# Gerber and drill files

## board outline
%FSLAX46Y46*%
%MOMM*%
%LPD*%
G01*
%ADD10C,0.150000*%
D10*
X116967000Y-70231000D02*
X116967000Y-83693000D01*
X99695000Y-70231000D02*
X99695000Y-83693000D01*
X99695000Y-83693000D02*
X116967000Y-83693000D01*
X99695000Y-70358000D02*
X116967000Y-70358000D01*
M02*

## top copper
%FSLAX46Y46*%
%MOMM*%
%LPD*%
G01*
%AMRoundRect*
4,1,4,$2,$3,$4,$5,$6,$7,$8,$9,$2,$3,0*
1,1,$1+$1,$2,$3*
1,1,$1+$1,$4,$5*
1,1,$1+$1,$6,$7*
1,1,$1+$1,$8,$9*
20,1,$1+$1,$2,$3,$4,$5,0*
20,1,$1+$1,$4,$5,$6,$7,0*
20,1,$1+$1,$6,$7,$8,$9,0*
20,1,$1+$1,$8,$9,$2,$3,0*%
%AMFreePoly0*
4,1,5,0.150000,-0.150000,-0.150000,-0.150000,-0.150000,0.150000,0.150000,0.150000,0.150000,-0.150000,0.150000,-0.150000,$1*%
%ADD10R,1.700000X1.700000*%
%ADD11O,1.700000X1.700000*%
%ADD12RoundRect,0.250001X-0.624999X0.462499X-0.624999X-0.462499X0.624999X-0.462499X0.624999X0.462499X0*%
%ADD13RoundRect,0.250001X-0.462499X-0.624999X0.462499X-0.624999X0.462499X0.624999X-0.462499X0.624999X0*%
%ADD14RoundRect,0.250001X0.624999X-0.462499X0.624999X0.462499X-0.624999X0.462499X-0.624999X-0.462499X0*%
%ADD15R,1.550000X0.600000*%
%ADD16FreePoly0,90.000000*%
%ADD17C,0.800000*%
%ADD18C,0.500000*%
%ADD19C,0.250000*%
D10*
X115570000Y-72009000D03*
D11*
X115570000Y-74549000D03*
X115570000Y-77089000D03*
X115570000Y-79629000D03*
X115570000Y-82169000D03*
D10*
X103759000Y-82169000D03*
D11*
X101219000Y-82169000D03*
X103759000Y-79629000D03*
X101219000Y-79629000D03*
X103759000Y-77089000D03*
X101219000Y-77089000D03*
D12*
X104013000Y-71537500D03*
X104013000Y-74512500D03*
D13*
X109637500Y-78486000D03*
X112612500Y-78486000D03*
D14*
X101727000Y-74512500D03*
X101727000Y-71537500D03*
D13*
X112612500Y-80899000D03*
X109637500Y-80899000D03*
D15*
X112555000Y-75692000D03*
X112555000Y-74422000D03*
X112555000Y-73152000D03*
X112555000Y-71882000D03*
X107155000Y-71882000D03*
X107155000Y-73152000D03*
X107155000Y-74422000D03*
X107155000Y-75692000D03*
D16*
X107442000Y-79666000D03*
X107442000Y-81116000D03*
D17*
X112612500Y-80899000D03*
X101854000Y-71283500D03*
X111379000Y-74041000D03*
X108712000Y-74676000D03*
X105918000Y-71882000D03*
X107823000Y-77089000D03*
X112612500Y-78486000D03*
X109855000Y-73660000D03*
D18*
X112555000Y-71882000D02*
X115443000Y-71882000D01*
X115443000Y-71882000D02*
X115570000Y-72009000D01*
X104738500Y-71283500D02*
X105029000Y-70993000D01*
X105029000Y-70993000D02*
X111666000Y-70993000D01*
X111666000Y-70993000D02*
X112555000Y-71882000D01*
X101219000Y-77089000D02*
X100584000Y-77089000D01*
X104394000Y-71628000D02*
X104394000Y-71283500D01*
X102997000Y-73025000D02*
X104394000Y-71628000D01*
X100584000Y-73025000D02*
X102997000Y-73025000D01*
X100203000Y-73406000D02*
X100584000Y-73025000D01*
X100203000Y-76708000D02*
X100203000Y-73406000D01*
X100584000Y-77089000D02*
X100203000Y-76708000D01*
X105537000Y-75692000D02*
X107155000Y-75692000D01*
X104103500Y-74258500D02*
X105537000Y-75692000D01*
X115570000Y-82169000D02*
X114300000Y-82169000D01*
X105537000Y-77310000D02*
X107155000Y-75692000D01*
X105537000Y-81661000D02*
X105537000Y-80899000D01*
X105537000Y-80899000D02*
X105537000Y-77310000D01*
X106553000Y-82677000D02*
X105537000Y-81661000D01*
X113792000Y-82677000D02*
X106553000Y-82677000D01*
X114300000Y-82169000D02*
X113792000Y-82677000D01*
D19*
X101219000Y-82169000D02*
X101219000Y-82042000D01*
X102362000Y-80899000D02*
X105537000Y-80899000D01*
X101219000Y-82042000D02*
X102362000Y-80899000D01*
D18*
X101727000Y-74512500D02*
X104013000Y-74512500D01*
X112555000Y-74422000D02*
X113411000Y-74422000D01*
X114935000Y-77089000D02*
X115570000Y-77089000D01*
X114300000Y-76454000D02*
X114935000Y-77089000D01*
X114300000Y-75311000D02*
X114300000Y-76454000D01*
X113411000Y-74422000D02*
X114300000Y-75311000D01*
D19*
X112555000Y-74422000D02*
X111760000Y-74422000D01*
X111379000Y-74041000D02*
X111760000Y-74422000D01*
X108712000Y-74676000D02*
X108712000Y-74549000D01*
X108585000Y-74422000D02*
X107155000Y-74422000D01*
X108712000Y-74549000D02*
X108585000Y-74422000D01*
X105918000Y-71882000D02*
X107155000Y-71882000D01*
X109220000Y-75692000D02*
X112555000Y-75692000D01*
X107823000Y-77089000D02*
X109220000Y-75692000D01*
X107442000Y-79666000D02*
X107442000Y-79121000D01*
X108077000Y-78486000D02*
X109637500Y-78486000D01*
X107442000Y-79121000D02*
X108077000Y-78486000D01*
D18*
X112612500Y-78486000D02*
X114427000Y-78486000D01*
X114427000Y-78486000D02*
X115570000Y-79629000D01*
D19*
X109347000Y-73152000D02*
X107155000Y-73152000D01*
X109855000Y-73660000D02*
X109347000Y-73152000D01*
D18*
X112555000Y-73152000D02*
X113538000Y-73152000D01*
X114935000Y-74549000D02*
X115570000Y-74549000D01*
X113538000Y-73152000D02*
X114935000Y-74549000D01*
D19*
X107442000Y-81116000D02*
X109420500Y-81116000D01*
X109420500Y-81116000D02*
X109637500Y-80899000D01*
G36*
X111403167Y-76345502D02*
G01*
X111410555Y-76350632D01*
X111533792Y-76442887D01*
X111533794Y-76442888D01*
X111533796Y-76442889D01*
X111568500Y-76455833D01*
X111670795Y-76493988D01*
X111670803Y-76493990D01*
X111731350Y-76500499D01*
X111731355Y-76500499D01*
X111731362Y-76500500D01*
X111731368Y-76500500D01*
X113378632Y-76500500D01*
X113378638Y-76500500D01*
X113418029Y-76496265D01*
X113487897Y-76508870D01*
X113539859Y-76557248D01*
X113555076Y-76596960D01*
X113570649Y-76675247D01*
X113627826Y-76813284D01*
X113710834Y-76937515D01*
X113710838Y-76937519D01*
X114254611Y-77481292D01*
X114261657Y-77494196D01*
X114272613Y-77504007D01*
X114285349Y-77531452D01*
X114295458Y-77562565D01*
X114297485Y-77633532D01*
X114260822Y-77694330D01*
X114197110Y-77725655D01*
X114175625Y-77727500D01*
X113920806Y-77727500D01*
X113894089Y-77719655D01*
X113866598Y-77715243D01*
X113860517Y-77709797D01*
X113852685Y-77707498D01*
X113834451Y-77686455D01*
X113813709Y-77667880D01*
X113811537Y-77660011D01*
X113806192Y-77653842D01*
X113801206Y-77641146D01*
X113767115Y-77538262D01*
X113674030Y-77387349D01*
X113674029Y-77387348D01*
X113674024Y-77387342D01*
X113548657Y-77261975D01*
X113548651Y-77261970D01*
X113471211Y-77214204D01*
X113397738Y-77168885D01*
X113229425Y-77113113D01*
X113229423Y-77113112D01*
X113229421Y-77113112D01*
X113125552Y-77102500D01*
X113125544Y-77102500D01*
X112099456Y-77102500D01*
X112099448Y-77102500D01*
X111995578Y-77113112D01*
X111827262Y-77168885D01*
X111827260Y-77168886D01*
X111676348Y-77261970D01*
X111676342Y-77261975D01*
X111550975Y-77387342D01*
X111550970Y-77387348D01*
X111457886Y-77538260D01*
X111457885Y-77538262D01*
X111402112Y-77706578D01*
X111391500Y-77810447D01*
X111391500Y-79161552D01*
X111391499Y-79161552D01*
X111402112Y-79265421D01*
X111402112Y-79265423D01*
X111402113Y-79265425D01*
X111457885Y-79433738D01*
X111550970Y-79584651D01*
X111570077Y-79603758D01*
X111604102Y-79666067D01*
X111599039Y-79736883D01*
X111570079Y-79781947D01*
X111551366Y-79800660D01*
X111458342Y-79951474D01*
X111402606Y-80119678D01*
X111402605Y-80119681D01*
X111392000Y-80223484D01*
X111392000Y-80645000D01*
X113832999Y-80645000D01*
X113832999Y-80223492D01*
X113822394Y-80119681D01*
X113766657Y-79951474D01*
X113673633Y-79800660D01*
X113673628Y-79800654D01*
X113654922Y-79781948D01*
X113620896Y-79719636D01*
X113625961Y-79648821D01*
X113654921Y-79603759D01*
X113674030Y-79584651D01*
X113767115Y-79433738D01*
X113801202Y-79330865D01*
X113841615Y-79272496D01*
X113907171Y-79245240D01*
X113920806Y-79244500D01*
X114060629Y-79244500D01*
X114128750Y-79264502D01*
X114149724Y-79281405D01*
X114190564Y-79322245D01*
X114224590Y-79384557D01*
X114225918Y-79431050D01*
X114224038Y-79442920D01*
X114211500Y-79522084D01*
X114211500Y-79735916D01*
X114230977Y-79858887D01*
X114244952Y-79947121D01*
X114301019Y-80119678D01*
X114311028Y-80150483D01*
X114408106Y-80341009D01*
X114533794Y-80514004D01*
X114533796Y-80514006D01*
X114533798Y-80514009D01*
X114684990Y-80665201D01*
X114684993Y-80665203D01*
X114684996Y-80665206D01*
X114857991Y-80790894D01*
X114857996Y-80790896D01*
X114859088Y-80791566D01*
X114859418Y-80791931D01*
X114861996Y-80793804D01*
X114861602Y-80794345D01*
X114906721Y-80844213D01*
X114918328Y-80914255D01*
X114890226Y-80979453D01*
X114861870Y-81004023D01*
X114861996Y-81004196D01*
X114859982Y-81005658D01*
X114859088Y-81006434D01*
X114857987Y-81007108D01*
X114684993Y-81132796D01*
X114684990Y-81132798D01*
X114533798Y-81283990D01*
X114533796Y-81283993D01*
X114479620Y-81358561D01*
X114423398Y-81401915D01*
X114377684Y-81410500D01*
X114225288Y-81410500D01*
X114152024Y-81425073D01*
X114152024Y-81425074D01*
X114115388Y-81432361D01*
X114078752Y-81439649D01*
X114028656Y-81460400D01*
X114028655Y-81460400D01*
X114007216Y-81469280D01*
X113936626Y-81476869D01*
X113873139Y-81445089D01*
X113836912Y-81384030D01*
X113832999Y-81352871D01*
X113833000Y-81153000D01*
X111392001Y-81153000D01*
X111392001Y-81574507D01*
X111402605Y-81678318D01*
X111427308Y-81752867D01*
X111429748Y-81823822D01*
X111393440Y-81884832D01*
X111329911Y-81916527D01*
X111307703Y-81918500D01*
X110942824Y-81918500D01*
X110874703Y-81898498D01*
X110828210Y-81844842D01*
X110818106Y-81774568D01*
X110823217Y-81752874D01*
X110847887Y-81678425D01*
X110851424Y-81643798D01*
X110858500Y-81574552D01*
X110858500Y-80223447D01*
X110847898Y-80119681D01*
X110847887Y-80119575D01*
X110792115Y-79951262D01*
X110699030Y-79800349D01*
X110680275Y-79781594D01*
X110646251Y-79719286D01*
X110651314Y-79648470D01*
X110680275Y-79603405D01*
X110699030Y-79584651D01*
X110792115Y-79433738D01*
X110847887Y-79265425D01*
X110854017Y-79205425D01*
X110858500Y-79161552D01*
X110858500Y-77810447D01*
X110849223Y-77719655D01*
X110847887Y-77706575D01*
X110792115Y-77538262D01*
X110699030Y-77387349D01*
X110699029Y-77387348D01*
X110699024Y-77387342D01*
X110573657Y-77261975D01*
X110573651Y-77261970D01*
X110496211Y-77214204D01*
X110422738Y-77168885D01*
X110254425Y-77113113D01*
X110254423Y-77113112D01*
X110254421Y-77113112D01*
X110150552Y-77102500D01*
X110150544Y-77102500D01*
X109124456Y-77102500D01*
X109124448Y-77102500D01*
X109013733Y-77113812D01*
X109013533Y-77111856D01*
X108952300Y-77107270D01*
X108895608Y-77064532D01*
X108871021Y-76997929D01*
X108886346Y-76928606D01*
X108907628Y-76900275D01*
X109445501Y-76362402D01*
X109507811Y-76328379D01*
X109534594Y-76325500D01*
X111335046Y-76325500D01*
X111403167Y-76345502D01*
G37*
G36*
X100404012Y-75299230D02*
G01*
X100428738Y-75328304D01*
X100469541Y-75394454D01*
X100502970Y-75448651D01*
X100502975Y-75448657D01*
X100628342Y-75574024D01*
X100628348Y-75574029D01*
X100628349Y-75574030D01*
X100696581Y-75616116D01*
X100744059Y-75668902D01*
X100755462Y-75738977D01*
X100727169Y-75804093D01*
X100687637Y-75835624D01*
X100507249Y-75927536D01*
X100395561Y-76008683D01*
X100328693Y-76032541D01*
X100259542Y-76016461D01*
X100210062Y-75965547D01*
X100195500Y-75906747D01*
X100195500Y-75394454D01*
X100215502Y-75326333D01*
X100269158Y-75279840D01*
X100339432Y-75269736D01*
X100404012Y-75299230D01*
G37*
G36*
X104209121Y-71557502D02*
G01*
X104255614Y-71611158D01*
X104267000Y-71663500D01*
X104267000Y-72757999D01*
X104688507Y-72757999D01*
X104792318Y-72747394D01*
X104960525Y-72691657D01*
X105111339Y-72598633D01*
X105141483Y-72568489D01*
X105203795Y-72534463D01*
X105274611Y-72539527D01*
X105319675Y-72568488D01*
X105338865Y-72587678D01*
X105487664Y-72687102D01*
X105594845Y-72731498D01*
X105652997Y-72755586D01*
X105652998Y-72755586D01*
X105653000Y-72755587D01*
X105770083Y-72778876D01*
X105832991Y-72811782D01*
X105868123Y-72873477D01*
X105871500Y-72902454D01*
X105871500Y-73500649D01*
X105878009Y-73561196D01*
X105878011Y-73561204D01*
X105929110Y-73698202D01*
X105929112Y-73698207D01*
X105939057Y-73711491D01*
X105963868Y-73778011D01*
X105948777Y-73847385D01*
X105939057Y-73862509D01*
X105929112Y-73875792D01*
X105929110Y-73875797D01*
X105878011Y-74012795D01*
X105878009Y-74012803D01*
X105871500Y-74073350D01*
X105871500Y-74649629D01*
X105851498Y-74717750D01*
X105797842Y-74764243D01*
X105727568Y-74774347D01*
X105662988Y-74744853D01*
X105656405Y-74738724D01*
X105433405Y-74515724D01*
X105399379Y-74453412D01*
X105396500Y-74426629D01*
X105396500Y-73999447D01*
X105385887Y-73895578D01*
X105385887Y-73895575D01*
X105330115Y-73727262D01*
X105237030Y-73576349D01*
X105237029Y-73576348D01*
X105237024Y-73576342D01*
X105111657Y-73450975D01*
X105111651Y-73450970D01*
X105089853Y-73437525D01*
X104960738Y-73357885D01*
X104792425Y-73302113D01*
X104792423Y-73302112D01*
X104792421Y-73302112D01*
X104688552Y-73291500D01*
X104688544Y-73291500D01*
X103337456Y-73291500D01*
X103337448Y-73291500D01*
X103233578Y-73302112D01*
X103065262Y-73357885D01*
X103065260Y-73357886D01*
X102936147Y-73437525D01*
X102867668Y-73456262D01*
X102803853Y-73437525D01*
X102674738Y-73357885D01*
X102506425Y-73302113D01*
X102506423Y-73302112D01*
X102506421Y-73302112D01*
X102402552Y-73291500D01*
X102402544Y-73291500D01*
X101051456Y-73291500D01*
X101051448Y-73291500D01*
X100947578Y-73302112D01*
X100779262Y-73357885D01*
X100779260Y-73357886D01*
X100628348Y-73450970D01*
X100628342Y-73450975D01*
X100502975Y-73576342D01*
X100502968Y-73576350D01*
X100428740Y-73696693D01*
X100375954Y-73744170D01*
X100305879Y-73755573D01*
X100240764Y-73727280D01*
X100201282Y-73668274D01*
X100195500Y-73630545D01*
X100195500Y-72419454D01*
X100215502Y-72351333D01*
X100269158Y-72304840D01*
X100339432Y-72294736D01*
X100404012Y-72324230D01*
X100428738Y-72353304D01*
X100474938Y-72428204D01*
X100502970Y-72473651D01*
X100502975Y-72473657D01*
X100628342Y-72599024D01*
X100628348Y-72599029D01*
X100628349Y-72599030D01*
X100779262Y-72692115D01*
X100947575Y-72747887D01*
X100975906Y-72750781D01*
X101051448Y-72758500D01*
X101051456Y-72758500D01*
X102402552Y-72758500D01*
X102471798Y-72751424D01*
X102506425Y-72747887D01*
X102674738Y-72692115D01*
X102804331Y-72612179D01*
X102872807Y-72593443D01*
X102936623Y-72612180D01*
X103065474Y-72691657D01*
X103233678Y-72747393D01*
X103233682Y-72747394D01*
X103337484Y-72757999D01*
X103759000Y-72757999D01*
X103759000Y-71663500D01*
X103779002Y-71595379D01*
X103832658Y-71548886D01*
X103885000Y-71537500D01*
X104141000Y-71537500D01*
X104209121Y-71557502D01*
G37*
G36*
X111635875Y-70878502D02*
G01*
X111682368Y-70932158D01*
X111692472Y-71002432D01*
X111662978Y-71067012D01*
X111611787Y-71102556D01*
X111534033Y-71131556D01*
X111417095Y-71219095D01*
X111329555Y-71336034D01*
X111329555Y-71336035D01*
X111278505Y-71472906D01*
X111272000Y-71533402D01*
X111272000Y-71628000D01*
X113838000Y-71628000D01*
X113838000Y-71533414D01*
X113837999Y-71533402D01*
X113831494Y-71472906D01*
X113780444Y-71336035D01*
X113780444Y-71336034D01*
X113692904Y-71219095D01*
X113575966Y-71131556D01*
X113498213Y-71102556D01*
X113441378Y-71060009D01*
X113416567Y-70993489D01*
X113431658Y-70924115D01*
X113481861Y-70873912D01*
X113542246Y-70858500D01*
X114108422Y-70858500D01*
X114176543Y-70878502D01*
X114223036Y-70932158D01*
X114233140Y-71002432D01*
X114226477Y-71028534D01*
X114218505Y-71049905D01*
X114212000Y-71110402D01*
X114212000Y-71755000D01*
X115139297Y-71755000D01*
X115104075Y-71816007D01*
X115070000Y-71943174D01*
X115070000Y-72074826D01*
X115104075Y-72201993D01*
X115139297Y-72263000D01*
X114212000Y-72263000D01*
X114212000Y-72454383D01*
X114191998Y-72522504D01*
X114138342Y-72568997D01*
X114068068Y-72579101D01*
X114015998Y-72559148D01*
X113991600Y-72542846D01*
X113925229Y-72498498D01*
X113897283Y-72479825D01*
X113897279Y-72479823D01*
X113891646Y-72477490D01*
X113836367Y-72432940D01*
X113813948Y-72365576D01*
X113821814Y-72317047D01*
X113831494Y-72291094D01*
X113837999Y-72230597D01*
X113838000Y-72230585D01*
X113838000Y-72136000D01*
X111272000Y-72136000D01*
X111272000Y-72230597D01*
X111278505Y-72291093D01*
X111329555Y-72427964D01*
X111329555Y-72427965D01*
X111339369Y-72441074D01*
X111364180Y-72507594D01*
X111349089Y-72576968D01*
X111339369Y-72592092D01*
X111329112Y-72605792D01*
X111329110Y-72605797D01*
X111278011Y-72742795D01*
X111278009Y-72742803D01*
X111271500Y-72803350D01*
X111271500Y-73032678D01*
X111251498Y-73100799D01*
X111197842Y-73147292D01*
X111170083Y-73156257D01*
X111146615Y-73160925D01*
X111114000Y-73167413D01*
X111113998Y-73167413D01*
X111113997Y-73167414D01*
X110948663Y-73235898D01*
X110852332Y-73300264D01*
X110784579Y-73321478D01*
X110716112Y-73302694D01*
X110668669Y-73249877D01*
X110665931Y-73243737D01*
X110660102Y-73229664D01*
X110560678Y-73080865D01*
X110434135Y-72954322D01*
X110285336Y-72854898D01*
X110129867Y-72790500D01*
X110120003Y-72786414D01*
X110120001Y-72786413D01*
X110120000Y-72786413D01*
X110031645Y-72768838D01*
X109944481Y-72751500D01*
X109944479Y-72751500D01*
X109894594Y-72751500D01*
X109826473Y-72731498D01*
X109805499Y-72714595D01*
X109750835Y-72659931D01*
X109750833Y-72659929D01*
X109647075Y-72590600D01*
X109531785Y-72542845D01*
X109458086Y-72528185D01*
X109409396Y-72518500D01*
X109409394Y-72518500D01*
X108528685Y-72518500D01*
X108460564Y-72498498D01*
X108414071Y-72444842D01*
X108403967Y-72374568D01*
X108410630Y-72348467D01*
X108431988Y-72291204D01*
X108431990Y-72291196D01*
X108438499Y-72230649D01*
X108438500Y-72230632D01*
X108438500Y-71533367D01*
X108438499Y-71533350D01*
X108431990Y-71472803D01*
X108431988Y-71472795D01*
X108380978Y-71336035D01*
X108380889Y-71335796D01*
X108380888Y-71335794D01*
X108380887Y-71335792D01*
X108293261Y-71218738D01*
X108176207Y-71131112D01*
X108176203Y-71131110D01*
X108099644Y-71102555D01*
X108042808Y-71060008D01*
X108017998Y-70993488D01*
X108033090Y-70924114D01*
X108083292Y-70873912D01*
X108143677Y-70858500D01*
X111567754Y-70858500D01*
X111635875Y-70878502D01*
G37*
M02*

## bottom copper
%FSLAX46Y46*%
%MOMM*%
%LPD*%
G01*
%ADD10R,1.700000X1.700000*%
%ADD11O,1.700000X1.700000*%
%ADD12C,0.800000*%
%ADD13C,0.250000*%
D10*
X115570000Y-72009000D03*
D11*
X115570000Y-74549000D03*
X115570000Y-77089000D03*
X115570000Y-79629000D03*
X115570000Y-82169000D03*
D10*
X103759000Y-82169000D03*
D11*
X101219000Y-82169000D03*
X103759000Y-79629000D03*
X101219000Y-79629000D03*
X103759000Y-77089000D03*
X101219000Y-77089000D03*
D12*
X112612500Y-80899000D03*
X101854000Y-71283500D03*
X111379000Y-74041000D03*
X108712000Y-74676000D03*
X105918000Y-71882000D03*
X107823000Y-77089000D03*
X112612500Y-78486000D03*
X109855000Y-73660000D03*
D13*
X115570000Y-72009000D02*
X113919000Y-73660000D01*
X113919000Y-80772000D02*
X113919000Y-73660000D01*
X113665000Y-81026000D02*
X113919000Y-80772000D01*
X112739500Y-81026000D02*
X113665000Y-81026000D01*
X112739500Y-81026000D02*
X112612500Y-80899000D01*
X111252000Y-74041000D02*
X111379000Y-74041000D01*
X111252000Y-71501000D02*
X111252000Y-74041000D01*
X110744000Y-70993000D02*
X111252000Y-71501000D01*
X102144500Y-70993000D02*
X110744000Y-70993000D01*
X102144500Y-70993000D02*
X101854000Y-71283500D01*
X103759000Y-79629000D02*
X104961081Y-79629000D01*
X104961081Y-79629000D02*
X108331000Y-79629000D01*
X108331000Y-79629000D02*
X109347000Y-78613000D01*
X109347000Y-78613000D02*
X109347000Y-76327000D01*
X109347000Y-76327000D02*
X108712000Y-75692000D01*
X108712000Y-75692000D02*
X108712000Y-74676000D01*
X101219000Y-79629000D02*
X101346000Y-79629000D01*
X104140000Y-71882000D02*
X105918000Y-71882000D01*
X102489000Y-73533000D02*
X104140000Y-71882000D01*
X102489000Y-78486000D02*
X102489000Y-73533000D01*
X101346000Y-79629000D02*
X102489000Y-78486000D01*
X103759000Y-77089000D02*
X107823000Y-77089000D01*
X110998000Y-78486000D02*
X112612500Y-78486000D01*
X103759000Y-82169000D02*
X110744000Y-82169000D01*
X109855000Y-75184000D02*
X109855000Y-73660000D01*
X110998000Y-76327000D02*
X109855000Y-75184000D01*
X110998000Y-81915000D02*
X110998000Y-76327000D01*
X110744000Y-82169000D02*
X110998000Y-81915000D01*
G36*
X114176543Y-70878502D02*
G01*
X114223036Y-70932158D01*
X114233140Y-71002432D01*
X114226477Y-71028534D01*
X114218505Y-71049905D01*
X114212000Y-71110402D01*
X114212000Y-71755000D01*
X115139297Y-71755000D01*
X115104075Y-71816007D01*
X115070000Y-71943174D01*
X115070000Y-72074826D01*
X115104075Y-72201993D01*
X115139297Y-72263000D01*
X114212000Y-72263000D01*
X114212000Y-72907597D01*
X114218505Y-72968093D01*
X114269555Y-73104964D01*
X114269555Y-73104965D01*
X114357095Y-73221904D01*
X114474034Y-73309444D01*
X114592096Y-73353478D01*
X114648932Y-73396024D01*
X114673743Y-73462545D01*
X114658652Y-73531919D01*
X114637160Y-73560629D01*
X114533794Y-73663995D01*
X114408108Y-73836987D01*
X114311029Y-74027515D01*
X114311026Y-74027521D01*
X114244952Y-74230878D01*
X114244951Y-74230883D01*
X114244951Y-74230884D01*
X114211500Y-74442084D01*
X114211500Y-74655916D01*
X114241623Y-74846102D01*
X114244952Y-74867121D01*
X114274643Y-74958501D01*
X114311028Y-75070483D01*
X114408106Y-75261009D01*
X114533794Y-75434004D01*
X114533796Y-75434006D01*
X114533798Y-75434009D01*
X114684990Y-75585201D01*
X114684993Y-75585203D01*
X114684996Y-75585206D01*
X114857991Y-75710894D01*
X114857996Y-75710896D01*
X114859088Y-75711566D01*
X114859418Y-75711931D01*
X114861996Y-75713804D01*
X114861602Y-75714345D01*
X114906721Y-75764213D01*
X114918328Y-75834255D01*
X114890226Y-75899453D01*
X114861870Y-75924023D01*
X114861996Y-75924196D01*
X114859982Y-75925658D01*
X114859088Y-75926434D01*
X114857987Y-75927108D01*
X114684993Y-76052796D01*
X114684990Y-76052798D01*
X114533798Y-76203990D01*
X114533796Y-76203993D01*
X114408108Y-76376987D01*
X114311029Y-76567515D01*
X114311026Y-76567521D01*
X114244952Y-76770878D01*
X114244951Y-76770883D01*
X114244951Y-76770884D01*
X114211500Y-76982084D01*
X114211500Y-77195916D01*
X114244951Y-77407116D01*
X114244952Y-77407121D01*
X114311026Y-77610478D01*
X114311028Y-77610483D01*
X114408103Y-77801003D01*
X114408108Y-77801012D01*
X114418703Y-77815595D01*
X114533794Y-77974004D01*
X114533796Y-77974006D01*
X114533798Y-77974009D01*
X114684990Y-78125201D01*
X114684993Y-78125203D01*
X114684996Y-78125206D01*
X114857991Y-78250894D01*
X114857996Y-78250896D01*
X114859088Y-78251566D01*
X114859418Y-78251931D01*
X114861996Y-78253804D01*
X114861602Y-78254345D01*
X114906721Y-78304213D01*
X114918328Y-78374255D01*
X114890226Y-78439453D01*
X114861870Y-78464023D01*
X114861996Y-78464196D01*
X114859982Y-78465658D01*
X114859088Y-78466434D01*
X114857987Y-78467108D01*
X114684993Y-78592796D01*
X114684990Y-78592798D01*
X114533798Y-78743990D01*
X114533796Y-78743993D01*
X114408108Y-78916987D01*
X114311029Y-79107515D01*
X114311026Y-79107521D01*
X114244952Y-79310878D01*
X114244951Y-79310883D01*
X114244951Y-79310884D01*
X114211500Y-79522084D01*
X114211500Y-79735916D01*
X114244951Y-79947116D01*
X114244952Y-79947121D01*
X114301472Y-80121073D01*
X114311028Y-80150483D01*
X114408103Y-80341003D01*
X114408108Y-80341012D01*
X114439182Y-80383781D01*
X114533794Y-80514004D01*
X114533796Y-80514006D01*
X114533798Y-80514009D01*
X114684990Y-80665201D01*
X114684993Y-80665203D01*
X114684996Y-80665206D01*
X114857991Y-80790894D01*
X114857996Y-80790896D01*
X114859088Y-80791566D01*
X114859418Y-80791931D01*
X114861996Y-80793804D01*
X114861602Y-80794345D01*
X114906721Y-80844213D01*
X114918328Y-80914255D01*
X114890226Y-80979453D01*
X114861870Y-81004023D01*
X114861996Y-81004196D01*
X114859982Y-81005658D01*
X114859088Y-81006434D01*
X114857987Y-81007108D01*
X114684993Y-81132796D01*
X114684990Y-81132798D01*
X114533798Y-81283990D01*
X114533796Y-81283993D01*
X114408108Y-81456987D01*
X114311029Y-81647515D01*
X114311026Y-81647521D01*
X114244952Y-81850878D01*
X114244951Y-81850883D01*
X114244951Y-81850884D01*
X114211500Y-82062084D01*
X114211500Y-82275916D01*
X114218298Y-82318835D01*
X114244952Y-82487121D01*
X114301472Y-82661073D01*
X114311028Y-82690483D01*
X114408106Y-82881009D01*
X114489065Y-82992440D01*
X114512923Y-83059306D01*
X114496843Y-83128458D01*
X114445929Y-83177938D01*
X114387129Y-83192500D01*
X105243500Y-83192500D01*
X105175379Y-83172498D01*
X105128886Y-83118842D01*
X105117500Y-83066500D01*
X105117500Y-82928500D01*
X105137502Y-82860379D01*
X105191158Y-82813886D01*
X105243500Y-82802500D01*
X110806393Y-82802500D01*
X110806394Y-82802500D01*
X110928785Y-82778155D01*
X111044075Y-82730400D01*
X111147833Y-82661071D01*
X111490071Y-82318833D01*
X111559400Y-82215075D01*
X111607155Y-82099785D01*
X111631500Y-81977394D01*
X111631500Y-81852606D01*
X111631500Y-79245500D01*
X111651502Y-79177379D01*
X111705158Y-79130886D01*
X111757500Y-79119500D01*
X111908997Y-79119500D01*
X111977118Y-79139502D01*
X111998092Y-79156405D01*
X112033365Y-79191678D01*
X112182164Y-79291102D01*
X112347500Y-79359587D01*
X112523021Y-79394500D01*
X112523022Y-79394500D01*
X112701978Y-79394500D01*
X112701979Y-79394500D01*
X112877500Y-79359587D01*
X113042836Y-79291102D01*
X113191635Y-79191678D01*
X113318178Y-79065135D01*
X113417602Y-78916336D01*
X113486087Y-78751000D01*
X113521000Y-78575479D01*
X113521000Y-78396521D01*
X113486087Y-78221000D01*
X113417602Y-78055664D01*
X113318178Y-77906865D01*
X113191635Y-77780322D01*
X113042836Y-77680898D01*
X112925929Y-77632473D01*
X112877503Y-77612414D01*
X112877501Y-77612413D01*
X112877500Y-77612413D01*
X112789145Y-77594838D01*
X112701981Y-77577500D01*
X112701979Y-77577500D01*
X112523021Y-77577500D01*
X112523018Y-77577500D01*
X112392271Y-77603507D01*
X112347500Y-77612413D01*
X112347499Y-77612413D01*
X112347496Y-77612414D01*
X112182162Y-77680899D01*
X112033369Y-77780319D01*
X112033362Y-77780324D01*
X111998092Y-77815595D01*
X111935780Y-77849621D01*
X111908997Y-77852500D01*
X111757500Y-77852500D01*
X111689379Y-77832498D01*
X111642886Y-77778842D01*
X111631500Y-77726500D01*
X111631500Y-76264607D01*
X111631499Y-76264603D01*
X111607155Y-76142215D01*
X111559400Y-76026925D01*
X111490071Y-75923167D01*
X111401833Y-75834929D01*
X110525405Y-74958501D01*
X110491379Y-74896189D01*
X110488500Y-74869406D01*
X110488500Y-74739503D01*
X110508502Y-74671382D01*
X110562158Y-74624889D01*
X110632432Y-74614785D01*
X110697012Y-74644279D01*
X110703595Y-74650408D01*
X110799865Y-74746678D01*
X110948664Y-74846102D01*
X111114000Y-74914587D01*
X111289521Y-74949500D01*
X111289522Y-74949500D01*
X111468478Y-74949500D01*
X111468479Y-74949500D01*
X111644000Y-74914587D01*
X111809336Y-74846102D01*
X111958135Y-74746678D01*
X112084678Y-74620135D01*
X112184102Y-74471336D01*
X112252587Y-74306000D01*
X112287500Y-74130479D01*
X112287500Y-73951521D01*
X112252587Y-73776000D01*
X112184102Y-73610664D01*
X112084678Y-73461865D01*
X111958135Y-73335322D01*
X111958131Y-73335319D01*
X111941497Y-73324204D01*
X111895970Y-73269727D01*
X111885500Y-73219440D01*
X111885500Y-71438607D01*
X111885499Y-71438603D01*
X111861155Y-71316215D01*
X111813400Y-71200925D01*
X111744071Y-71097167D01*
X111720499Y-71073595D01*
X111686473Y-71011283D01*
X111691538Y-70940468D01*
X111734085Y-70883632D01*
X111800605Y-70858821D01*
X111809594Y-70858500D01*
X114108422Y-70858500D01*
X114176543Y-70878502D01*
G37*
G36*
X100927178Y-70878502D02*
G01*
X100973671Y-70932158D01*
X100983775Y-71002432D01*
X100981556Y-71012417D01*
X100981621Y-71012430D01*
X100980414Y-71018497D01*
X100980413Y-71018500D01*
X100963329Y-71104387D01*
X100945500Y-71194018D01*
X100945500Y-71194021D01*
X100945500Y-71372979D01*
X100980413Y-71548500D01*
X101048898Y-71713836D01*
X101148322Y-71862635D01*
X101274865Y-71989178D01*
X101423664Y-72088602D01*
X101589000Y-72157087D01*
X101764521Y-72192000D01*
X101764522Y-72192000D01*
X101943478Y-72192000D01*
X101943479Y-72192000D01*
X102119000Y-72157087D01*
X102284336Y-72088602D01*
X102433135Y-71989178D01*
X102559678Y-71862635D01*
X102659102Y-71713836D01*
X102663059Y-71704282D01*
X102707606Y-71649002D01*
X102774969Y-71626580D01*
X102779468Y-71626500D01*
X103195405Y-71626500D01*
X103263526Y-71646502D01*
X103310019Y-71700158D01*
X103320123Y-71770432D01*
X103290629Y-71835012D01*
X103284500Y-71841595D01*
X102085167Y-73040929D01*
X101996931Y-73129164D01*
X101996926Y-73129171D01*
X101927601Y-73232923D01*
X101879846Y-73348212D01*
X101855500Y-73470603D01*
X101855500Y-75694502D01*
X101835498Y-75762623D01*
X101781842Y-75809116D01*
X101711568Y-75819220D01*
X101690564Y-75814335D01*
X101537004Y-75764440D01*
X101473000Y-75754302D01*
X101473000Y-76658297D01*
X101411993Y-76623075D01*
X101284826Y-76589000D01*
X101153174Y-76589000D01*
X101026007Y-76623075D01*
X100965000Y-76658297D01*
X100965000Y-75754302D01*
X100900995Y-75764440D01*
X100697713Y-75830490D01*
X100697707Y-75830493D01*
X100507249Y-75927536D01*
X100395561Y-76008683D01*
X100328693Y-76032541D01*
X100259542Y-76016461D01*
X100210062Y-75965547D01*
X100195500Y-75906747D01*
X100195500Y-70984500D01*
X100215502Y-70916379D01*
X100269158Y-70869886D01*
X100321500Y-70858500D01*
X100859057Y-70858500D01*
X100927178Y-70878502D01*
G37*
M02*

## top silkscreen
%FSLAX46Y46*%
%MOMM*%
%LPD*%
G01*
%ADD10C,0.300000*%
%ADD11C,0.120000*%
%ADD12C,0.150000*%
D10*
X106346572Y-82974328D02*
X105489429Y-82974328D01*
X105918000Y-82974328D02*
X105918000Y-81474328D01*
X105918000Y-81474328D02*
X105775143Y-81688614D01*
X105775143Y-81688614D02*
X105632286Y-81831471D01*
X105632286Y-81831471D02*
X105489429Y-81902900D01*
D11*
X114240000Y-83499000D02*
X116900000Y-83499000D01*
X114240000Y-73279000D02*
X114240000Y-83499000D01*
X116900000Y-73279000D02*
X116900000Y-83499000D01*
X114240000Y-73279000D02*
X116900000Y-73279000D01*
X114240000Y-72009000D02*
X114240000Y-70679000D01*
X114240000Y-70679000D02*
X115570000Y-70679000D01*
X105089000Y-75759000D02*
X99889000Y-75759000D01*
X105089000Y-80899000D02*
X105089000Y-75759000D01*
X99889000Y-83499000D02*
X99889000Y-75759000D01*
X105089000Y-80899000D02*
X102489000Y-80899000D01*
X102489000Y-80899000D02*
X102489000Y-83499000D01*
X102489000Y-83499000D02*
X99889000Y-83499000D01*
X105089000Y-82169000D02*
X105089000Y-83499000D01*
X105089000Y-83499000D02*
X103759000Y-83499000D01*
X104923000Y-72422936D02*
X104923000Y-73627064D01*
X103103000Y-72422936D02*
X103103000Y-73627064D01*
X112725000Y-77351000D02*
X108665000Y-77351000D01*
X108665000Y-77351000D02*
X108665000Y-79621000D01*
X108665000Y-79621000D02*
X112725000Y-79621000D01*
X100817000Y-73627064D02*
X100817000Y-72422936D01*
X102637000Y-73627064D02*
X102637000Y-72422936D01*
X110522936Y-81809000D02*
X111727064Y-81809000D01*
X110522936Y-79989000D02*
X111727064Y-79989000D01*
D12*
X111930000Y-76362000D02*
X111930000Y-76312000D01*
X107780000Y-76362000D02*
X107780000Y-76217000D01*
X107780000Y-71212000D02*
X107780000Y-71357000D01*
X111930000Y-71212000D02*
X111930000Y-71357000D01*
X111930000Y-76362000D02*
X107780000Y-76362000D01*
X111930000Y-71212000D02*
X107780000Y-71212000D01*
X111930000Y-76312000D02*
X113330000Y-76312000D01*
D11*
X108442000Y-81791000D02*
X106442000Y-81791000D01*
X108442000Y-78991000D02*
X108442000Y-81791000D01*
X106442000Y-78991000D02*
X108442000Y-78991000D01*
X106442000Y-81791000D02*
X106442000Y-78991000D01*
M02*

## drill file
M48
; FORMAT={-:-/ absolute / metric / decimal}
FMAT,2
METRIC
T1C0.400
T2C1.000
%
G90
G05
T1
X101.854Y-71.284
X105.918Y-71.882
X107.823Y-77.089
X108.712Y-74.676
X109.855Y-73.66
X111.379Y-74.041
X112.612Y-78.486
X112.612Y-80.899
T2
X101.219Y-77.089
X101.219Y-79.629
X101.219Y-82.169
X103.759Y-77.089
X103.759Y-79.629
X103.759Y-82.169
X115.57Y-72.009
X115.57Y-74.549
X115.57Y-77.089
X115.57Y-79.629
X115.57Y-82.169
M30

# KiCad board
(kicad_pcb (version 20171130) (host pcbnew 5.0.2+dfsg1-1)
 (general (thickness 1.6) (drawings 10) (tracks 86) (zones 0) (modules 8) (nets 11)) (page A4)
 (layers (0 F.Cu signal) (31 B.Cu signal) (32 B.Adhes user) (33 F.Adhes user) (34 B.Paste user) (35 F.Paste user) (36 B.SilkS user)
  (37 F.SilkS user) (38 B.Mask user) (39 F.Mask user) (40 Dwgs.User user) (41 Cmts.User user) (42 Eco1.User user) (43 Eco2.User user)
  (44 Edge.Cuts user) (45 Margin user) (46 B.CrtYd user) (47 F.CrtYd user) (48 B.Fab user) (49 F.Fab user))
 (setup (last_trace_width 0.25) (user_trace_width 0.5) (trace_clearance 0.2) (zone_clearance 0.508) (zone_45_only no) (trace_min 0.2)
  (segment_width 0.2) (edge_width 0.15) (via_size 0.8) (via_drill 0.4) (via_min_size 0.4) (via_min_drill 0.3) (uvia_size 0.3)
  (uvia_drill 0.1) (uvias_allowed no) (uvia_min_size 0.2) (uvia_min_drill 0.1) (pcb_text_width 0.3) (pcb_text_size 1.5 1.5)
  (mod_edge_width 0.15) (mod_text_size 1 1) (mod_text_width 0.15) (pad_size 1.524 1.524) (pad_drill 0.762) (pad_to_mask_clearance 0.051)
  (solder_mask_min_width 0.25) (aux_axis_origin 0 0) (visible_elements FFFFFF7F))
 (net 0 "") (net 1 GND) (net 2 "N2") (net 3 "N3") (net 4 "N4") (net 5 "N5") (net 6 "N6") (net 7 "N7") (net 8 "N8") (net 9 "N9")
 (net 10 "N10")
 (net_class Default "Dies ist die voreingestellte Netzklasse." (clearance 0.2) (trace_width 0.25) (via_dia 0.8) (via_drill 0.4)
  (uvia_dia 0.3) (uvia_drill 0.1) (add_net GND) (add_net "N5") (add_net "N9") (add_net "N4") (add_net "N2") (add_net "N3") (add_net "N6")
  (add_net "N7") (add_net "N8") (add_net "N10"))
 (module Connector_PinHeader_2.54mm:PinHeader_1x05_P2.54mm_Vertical (layer F.Cu) (at 115.57 72.009)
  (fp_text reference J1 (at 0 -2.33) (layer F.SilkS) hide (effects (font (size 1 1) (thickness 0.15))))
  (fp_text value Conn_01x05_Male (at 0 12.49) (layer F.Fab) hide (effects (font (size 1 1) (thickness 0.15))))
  (fp_line (start -1.33 11.49) (end 1.33 11.49) (layer F.SilkS) (width 0.12))
  (fp_line (start -1.33 1.27) (end -1.33 11.49) (layer F.SilkS) (width 0.12))
  (fp_line (start 1.33 1.27) (end 1.33 11.49) (layer F.SilkS) (width 0.12))
  (fp_line (start -1.33 1.27) (end 1.33 1.27) (layer F.SilkS) (width 0.12))
  (fp_line (start -1.33 0) (end -1.33 -1.33) (layer F.SilkS) (width 0.12))
  (fp_line (start -1.33 -1.33) (end 0 -1.33) (layer F.SilkS) (width 0.12))
  (pad 1 thru_hole rect (at 0 0) (size 1.7 1.7) (drill 1) (layers *.Cu *.Mask) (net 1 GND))
  (pad 2 thru_hole oval (at 0 2.54) (size 1.7 1.7) (drill 1) (layers *.Cu *.Mask) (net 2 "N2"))
  (pad 3 thru_hole oval (at 0 5.08) (size 1.7 1.7) (drill 1) (layers *.Cu *.Mask) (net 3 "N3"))
  (pad 4 thru_hole oval (at 0 7.62) (size 1.7 1.7) (drill 1) (layers *.Cu *.Mask) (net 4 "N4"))
  (pad 5 thru_hole oval (at 0 10.16) (size 1.7 1.7) (drill 1) (layers *.Cu *.Mask) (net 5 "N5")))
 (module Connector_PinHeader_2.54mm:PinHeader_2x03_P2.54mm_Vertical (layer F.Cu) (at 103.759 82.169 180)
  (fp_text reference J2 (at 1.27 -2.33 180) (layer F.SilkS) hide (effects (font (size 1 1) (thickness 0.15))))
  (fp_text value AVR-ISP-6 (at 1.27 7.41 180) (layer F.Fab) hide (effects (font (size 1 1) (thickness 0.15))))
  (fp_line (start -1.33 6.41) (end 3.87 6.41) (layer F.SilkS) (width 0.12))
  (fp_line (start -1.33 1.27) (end -1.33 6.41) (layer F.SilkS) (width 0.12))
  (fp_line (start 3.87 -1.33) (end 3.87 6.41) (layer F.SilkS) (width 0.12))
  (fp_line (start -1.33 1.27) (end 1.27 1.27) (layer F.SilkS) (width 0.12))
  (fp_line (start 1.27 1.27) (end 1.27 -1.33) (layer F.SilkS) (width 0.12))
  (fp_line (start 1.27 -1.33) (end 3.87 -1.33) (layer F.SilkS) (width 0.12))
  (fp_line (start -1.33 0) (end -1.33 -1.33) (layer F.SilkS) (width 0.12))
  (fp_line (start -1.33 -1.33) (end 0 -1.33) (layer F.SilkS) (width 0.12))
  (pad 1 thru_hole rect (at 0 0 180) (size 1.7 1.7) (drill 1) (layers *.Cu *.Mask) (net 4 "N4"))
  (pad 2 thru_hole oval (at 2.54 0 180) (size 1.7 1.7) (drill 1) (layers *.Cu *.Mask) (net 5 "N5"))
  (pad 3 thru_hole oval (at 0 2.54 180) (size 1.7 1.7) (drill 1) (layers *.Cu *.Mask) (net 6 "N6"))
  (pad 4 thru_hole oval (at 2.54 2.54 180) (size 1.7 1.7) (drill 1) (layers *.Cu *.Mask) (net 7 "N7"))
  (pad 5 thru_hole oval (at 0 5.08 180) (size 1.7 1.7) (drill 1) (layers *.Cu *.Mask) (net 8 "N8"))
  (pad 6 thru_hole oval (at 2.54 5.08 180) (size 1.7 1.7) (drill 1) (layers *.Cu *.Mask) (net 1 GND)))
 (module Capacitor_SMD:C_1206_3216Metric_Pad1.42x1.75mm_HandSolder (layer F.Cu) (at 104.013 73.025 270)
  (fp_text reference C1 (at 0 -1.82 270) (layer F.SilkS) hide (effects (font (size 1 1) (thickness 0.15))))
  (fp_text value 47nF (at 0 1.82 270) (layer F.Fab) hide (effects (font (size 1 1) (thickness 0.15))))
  (fp_line (start -0.602064 -0.91) (end 0.602064 -0.91) (layer F.SilkS) (width 0.12))
  (fp_line (start -0.602064 0.91) (end 0.602064 0.91) (layer F.SilkS) (width 0.12))
  (pad 1 smd roundrect (at -1.4875 0 270) (size 1.425 1.75) (layers F.Cu F.Paste F.Mask) (roundrect_rratio 0.175439) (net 1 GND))
  (pad 2 smd roundrect (at 1.4875 0 270) (size 1.425 1.75) (layers F.Cu F.Paste F.Mask) (roundrect_rratio 0.175439) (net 5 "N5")))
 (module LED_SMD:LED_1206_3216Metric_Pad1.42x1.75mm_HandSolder (layer F.Cu) (at 111.125 78.486)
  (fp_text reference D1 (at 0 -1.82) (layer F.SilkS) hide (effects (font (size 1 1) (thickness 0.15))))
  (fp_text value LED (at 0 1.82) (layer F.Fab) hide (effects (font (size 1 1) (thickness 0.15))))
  (fp_line (start 1.6 -1.135) (end -2.46 -1.135) (layer F.SilkS) (width 0.12))
  (fp_line (start -2.46 -1.135) (end -2.46 1.135) (layer F.SilkS) (width 0.12))
  (fp_line (start -2.46 1.135) (end 1.6 1.135) (layer F.SilkS) (width 0.12))
  (pad 1 smd roundrect (at -1.4875 0) (size 1.425 1.75) (layers F.Cu F.Paste F.Mask) (roundrect_rratio 0.175439) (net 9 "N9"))
  (pad 2 smd roundrect (at 1.4875 0) (size 1.425 1.75) (layers F.Cu F.Paste F.Mask) (roundrect_rratio 0.175439) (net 4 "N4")))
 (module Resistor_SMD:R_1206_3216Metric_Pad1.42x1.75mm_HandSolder (layer F.Cu) (at 101.727 73.025 90)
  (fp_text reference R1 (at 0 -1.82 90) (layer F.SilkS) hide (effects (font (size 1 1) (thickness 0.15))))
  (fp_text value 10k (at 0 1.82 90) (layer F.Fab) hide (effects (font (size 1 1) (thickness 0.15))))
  (fp_line (start -0.602064 -0.91) (end 0.602064 -0.91) (layer F.SilkS) (width 0.12))
  (fp_line (start -0.602064 0.91) (end 0.602064 0.91) (layer F.SilkS) (width 0.12))
  (pad 1 smd roundrect (at -1.4875 0 90) (size 1.425 1.75) (layers F.Cu F.Paste F.Mask) (roundrect_rratio 0.175439) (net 5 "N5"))
  (pad 2 smd roundrect (at 1.4875 0 90) (size 1.425 1.75) (layers F.Cu F.Paste F.Mask) (roundrect_rratio 0.175439) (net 3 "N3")))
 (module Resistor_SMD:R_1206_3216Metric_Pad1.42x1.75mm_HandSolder (layer F.Cu) (at 111.125 80.899)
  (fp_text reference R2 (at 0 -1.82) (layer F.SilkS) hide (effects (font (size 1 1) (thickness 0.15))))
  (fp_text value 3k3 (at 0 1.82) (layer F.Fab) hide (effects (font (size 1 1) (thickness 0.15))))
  (fp_line (start -0.602064 0.91) (end 0.602064 0.91) (layer F.SilkS) (width 0.12))
  (fp_line (start -0.602064 -0.91) (end 0.602064 -0.91) (layer F.SilkS) (width 0.12))
  (pad 2 smd roundrect (at 1.4875 0) (size 1.425 1.75) (layers F.Cu F.Paste F.Mask) (roundrect_rratio 0.175439) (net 1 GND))
  (pad 1 smd roundrect (at -1.4875 0) (size 1.425 1.75) (layers F.Cu F.Paste F.Mask) (roundrect_rratio 0.175439) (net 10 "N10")))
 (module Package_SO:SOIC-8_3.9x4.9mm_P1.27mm (layer F.Cu) (at 109.855 73.787 180)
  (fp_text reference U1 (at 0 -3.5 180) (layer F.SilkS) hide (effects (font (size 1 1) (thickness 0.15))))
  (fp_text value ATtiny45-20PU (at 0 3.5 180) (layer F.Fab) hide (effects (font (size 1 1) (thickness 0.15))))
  (fp_line (start -2.075 -2.575) (end -2.075 -2.525) (layer F.SilkS) (width 0.15))
  (fp_line (start 2.075 -2.575) (end 2.075 -2.43) (layer F.SilkS) (width 0.15))
  (fp_line (start 2.075 2.575) (end 2.075 2.43) (layer F.SilkS) (width 0.15))
  (fp_line (start -2.075 2.575) (end -2.075 2.43) (layer F.SilkS) (width 0.15))
  (fp_line (start -2.075 -2.575) (end 2.075 -2.575) (layer F.SilkS) (width 0.15))
  (fp_line (start -2.075 2.575) (end 2.075 2.575) (layer F.SilkS) (width 0.15))
  (fp_line (start -2.075 -2.525) (end -3.475 -2.525) (layer F.SilkS) (width 0.15))
  (pad 1 smd rect (at -2.7 -1.905 180) (size 1.55 0.6) (layers F.Cu F.Paste F.Mask) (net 8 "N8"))
  (pad 2 smd rect (at -2.7 -0.635 180) (size 1.55 0.6) (layers F.Cu F.Paste F.Mask) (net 3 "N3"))
  (pad 3 smd rect (at -2.7 0.635 180) (size 1.55 0.6) (layers F.Cu F.Paste F.Mask) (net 2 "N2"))
  (pad 4 smd rect (at -2.7 1.905 180) (size 1.55 0.6) (layers F.Cu F.Paste F.Mask) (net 1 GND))
  (pad 5 smd rect (at 2.7 1.905 180) (size 1.55 0.6) (layers F.Cu F.Paste F.Mask) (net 7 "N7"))
  (pad 6 smd rect (at 2.7 0.635 180) (size 1.55 0.6) (layers F.Cu F.Paste F.Mask) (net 4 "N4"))
  (pad 7 smd rect (at 2.7 -0.635 180) (size 1.55 0.6) (layers F.Cu F.Paste F.Mask) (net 6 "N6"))
  (pad 8 smd rect (at 2.7 -1.905 180) (size 1.55 0.6) (layers F.Cu F.Paste F.Mask) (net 5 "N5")))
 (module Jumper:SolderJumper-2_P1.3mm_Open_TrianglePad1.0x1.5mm (layer F.Cu) (at 107.442 80.391 90)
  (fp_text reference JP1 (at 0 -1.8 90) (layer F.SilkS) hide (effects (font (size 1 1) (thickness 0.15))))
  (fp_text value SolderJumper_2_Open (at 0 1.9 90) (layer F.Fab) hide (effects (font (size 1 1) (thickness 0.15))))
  (fp_line (start -1.4 1) (end -1.4 -1) (layer F.SilkS) (width 0.12))
  (fp_line (start 1.4 1) (end -1.4 1) (layer F.SilkS) (width 0.12))
  (fp_line (start 1.4 -1) (end 1.4 1) (layer F.SilkS) (width 0.12))
  (fp_line (start -1.4 -1) (end 1.4 -1) (layer F.SilkS) (width 0.12))
  (pad 2 smd custom (at 0.725 0 90) (size 0.3 0.3) (layers F.Cu F.Mask) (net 9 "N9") (zone_connect 0)
   (options (clearance outline) (anchor rect)) (primitives))
  (pad 1 smd custom (at -0.725 0 90) (size 0.3 0.3) (layers F.Cu F.Mask) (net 10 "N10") (zone_connect 0)
   (options (clearance outline) (anchor rect)) (primitives)))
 (gr_line (start 116.967 70.231) (end 116.967 83.693) (angle 90) (layer Edge.Cuts) (width 0.15))
 (gr_line (start 99.695 70.231) (end 99.695 83.693) (angle 90) (layer Edge.Cuts) (width 0.15))
 (gr_line (start 99.695 83.693) (end 116.967 83.693) (angle 90) (layer Edge.Cuts) (width 0.15))
 (gr_line (start 99.695 70.358) (end 116.967 70.358) (angle 90) (layer Edge.Cuts) (width 0.15))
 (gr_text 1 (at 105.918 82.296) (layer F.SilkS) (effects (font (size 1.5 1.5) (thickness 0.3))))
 (segment (start 112.555 71.882) (end 115.443 71.882) (width 0.5) (layer F.Cu) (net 1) (status C00000))
 (segment (start 115.443 71.882) (end 115.57 72.009) (width 0.5) (layer F.Cu) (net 1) (status C00000))
 (segment (start 104.7385 71.2835) (end 105.029 70.993) (width 0.5) (layer F.Cu) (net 1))
 (segment (start 105.029 70.993) (end 111.666 70.993) (width 0.5) (layer F.Cu) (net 1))
 (segment (start 111.666 70.993) (end 112.555 71.882) (width 0.5) (layer F.Cu) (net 1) (status 800000))
 (segment (start 101.219 77.089) (end 100.584 77.089) (width 0.5) (layer F.Cu) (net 1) (status C00000))
 (segment (start 104.394 71.628) (end 104.394 71.2835) (width 0.5) (layer F.Cu) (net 1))
 (segment (start 102.997 73.025) (end 104.394 71.628) (width 0.5) (layer F.Cu) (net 1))
 (segment (start 100.584 73.025) (end 102.997 73.025) (width 0.5) (layer F.Cu) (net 1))
 (segment (start 100.203 73.406) (end 100.584 73.025) (width 0.5) (layer F.Cu) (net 1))
 (segment (start 100.203 76.708) (end 100.203 73.406) (width 0.5) (layer F.Cu) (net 1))
 (segment (start 100.584 77.089) (end 100.203 76.708) (width 0.5) (layer F.Cu) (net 1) (status 400000))
 (via (at 112.6125 80.899) (size 0.8) (drill 0.4) (layers F.Cu B.Cu) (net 1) (status C00000))
 (segment (start 115.57 72.009) (end 113.919 73.66) (width 0.25) (layer B.Cu) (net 1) (status 400000))
 (segment (start 113.919 80.772) (end 113.919 73.66) (width 0.25) (layer B.Cu) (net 1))
 (segment (start 113.665 81.026) (end 113.919 80.772) (width 0.25) (layer B.Cu) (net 1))
 (segment (start 112.7395 81.026) (end 113.665 81.026) (width 0.25) (layer B.Cu) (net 1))
 (segment (start 112.7395 81.026) (end 112.6125 80.899) (width 0.25) (layer B.Cu) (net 1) (status 800000))
 (segment (start 105.537 75.692) (end 107.155 75.692) (width 0.5) (layer F.Cu) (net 5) (status 800000))
 (segment (start 104.1035 74.2585) (end 105.537 75.692) (width 0.5) (layer F.Cu) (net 5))
 (segment (start 115.57 82.169) (end 114.3 82.169) (width 0.5) (layer F.Cu) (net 5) (status 400000))
 (segment (start 105.537 77.31) (end 107.155 75.692) (width 0.5) (layer F.Cu) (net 5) (status 800000))
 (segment (start 105.537 81.661) (end 105.537 80.899) (width 0.5) (layer F.Cu) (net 5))
 (segment (start 105.537 80.899) (end 105.537 77.31) (width 0.5) (layer F.Cu) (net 5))
 (segment (start 106.553 82.677) (end 105.537 81.661) (width 0.5) (layer F.Cu) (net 5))
 (segment (start 113.792 82.677) (end 106.553 82.677) (width 0.5) (layer F.Cu) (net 5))
 (segment (start 114.3 82.169) (end 113.792 82.677) (width 0.5) (layer F.Cu) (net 5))
 (segment (start 101.219 82.169) (end 101.219 82.042) (width 0.25) (layer F.Cu) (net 5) (status C00000))
 (segment (start 102.362 80.899) (end 105.537 80.899) (width 0.25) (layer F.Cu) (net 5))
 (segment (start 101.219 82.042) (end 102.362 80.899) (width 0.25) (layer F.Cu) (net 5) (status 400000))
 (segment (start 101.727 74.5125) (end 104.013 74.5125) (width 0.5) (layer F.Cu) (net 5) (status C00000))
 (segment (start 112.555 74.422) (end 113.411 74.422) (width 0.5) (layer F.Cu) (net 3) (status 400000))
 (segment (start 114.935 77.089) (end 115.57 77.089) (width 0.5) (layer F.Cu) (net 3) (status C00000))
 (segment (start 114.3 76.454) (end 114.935 77.089) (width 0.5) (layer F.Cu) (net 3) (status 800000))
 (segment (start 114.3 75.311) (end 114.3 76.454) (width 0.5) (layer F.Cu) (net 3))
 (segment (start 113.411 74.422) (end 114.3 75.311) (width 0.5) (layer F.Cu) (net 3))
 (via (at 101.854 71.2835) (size 0.8) (drill 0.4) (layers F.Cu B.Cu) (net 3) (status C00000))
 (segment (start 112.555 74.422) (end 111.76 74.422) (width 0.25) (layer F.Cu) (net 3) (status 400000))
 (segment (start 111.379 74.041) (end 111.76 74.422) (width 0.25) (layer F.Cu) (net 3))
 (via (at 111.379 74.041) (size 0.8) (drill 0.4) (layers F.Cu B.Cu) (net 3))
 (segment (start 111.252 74.041) (end 111.379 74.041) (width 0.25) (layer B.Cu) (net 3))
 (segment (start 111.252 71.501) (end 111.252 74.041) (width 0.25) (layer B.Cu) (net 3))
 (segment (start 110.744 70.993) (end 111.252 71.501) (width 0.25) (layer B.Cu) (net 3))
 (segment (start 102.1445 70.993) (end 110.744 70.993) (width 0.25) (layer B.Cu) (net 3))
 (segment (start 102.1445 70.993) (end 101.854 71.2835) (width 0.25) (layer B.Cu) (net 3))
 (segment (start 103.759 79.629) (end 104.961081 79.629) (width 0.25) (layer B.Cu) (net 6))
 (segment (start 104.961081 79.629) (end 108.331 79.629) (width 0.25) (layer B.Cu) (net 6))
 (segment (start 108.331 79.629) (end 109.347 78.613) (width 0.25) (layer B.Cu) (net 6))
 (segment (start 109.347 78.613) (end 109.347 76.327) (width 0.25) (layer B.Cu) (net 6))
 (via (at 108.712 74.676) (size 0.8) (drill 0.4) (layers F.Cu B.Cu) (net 6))
 (segment (start 109.347 76.327) (end 108.712 75.692) (width 0.25) (layer B.Cu) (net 6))
 (segment (start 108.712 75.692) (end 108.712 74.676) (width 0.25) (layer B.Cu) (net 6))
 (segment (start 108.712 74.676) (end 108.712 74.549) (width 0.25) (layer F.Cu) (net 6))
 (segment (start 108.585 74.422) (end 107.155 74.422) (width 0.25) (layer F.Cu) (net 6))
 (segment (start 108.712 74.549) (end 108.585 74.422) (width 0.25) (layer F.Cu) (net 6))
 (segment (start 101.219 79.629) (end 101.346 79.629) (width 0.25) (layer B.Cu) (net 7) (status C00000))
 (segment (start 105.918 71.882) (end 107.155 71.882) (width 0.25) (layer F.Cu) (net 7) (status 800000))
 (via (at 105.918 71.882) (size 0.8) (drill 0.4) (layers F.Cu B.Cu) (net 7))
 (segment (start 104.14 71.882) (end 105.918 71.882) (width 0.25) (layer B.Cu) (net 7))
 (segment (start 102.489 73.533) (end 104.14 71.882) (width 0.25) (layer B.Cu) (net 7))
 (segment (start 102.489 78.486) (end 102.489 73.533) (width 0.25) (layer B.Cu) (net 7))
 (segment (start 101.346 79.629) (end 102.489 78.486) (width 0.25) (layer B.Cu) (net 7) (status 400000))
 (segment (start 103.759 77.089) (end 107.823 77.089) (width 0.25) (layer B.Cu) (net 8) (status 400000))
 (segment (start 109.22 75.692) (end 112.555 75.692) (width 0.25) (layer F.Cu) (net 8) (status 800000))
 (segment (start 107.823 77.089) (end 109.22 75.692) (width 0.25) (layer F.Cu) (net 8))
 (via (at 107.823 77.089) (size 0.8) (drill 0.4) (layers F.Cu B.Cu) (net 8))
 (segment (start 107.442 79.666) (end 107.442 79.121) (width 0.25) (layer F.Cu) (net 9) (status 400000))
 (segment (start 108.077 78.486) (end 109.6375 78.486) (width 0.25) (layer F.Cu) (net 9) (status 800000))
 (segment (start 107.442 79.121) (end 108.077 78.486) (width 0.25) (layer F.Cu) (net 9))
 (segment (start 112.6125 78.486) (end 114.427 78.486) (width 0.5) (layer F.Cu) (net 4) (status 400000))
 (segment (start 110.998 78.486) (end 112.6125 78.486) (width 0.25) (layer B.Cu) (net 4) (status 800000))
 (via (at 112.6125 78.486) (size 0.8) (drill 0.4) (layers F.Cu B.Cu) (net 4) (status C00000))
 (segment (start 114.427 78.486) (end 115.57 79.629) (width 0.5) (layer F.Cu) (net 4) (status 800000))
 (segment (start 103.759 82.169) (end 110.744 82.169) (width 0.25) (layer B.Cu) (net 4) (status 400000))
 (segment (start 109.347 73.152) (end 107.155 73.152) (width 0.25) (layer F.Cu) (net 4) (status 800000))
 (segment (start 109.855 73.66) (end 109.347 73.152) (width 0.25) (layer F.Cu) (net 4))
 (via (at 109.855 73.66) (size 0.8) (drill 0.4) (layers F.Cu B.Cu) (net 4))
 (segment (start 109.855 75.184) (end 109.855 73.66) (width 0.25) (layer B.Cu) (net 4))
 (segment (start 110.998 76.327) (end 109.855 75.184) (width 0.25) (layer B.Cu) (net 4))
 (segment (start 110.998 81.915) (end 110.998 76.327) (width 0.25) (layer B.Cu) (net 4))
 (segment (start 110.744 82.169) (end 110.998 81.915) (width 0.25) (layer B.Cu) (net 4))
 (segment (start 112.555 73.152) (end 113.538 73.152) (width 0.5) (layer F.Cu) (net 2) (status 400000))
 (segment (start 114.935 74.549) (end 115.57 74.549) (width 0.5) (layer F.Cu) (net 2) (status C00000))
 (segment (start 113.538 73.152) (end 114.935 74.549) (width 0.5) (layer F.Cu) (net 2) (status 800000))
 (segment (start 107.442 81.116) (end 109.4205 81.116) (width 0.25) (layer F.Cu) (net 10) (status C00000))
 (segment (start 109.4205 81.116) (end 109.6375 80.899) (width 0.25) (layer F.Cu) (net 10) (status C00000))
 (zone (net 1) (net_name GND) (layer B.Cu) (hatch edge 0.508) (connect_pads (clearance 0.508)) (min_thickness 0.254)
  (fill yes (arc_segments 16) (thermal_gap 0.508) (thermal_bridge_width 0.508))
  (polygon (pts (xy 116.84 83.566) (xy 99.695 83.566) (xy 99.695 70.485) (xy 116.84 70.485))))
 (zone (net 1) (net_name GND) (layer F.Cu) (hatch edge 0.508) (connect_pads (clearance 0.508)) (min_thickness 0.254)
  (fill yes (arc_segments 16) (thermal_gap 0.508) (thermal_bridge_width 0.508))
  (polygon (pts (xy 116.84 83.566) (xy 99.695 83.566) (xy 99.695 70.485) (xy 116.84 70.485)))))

